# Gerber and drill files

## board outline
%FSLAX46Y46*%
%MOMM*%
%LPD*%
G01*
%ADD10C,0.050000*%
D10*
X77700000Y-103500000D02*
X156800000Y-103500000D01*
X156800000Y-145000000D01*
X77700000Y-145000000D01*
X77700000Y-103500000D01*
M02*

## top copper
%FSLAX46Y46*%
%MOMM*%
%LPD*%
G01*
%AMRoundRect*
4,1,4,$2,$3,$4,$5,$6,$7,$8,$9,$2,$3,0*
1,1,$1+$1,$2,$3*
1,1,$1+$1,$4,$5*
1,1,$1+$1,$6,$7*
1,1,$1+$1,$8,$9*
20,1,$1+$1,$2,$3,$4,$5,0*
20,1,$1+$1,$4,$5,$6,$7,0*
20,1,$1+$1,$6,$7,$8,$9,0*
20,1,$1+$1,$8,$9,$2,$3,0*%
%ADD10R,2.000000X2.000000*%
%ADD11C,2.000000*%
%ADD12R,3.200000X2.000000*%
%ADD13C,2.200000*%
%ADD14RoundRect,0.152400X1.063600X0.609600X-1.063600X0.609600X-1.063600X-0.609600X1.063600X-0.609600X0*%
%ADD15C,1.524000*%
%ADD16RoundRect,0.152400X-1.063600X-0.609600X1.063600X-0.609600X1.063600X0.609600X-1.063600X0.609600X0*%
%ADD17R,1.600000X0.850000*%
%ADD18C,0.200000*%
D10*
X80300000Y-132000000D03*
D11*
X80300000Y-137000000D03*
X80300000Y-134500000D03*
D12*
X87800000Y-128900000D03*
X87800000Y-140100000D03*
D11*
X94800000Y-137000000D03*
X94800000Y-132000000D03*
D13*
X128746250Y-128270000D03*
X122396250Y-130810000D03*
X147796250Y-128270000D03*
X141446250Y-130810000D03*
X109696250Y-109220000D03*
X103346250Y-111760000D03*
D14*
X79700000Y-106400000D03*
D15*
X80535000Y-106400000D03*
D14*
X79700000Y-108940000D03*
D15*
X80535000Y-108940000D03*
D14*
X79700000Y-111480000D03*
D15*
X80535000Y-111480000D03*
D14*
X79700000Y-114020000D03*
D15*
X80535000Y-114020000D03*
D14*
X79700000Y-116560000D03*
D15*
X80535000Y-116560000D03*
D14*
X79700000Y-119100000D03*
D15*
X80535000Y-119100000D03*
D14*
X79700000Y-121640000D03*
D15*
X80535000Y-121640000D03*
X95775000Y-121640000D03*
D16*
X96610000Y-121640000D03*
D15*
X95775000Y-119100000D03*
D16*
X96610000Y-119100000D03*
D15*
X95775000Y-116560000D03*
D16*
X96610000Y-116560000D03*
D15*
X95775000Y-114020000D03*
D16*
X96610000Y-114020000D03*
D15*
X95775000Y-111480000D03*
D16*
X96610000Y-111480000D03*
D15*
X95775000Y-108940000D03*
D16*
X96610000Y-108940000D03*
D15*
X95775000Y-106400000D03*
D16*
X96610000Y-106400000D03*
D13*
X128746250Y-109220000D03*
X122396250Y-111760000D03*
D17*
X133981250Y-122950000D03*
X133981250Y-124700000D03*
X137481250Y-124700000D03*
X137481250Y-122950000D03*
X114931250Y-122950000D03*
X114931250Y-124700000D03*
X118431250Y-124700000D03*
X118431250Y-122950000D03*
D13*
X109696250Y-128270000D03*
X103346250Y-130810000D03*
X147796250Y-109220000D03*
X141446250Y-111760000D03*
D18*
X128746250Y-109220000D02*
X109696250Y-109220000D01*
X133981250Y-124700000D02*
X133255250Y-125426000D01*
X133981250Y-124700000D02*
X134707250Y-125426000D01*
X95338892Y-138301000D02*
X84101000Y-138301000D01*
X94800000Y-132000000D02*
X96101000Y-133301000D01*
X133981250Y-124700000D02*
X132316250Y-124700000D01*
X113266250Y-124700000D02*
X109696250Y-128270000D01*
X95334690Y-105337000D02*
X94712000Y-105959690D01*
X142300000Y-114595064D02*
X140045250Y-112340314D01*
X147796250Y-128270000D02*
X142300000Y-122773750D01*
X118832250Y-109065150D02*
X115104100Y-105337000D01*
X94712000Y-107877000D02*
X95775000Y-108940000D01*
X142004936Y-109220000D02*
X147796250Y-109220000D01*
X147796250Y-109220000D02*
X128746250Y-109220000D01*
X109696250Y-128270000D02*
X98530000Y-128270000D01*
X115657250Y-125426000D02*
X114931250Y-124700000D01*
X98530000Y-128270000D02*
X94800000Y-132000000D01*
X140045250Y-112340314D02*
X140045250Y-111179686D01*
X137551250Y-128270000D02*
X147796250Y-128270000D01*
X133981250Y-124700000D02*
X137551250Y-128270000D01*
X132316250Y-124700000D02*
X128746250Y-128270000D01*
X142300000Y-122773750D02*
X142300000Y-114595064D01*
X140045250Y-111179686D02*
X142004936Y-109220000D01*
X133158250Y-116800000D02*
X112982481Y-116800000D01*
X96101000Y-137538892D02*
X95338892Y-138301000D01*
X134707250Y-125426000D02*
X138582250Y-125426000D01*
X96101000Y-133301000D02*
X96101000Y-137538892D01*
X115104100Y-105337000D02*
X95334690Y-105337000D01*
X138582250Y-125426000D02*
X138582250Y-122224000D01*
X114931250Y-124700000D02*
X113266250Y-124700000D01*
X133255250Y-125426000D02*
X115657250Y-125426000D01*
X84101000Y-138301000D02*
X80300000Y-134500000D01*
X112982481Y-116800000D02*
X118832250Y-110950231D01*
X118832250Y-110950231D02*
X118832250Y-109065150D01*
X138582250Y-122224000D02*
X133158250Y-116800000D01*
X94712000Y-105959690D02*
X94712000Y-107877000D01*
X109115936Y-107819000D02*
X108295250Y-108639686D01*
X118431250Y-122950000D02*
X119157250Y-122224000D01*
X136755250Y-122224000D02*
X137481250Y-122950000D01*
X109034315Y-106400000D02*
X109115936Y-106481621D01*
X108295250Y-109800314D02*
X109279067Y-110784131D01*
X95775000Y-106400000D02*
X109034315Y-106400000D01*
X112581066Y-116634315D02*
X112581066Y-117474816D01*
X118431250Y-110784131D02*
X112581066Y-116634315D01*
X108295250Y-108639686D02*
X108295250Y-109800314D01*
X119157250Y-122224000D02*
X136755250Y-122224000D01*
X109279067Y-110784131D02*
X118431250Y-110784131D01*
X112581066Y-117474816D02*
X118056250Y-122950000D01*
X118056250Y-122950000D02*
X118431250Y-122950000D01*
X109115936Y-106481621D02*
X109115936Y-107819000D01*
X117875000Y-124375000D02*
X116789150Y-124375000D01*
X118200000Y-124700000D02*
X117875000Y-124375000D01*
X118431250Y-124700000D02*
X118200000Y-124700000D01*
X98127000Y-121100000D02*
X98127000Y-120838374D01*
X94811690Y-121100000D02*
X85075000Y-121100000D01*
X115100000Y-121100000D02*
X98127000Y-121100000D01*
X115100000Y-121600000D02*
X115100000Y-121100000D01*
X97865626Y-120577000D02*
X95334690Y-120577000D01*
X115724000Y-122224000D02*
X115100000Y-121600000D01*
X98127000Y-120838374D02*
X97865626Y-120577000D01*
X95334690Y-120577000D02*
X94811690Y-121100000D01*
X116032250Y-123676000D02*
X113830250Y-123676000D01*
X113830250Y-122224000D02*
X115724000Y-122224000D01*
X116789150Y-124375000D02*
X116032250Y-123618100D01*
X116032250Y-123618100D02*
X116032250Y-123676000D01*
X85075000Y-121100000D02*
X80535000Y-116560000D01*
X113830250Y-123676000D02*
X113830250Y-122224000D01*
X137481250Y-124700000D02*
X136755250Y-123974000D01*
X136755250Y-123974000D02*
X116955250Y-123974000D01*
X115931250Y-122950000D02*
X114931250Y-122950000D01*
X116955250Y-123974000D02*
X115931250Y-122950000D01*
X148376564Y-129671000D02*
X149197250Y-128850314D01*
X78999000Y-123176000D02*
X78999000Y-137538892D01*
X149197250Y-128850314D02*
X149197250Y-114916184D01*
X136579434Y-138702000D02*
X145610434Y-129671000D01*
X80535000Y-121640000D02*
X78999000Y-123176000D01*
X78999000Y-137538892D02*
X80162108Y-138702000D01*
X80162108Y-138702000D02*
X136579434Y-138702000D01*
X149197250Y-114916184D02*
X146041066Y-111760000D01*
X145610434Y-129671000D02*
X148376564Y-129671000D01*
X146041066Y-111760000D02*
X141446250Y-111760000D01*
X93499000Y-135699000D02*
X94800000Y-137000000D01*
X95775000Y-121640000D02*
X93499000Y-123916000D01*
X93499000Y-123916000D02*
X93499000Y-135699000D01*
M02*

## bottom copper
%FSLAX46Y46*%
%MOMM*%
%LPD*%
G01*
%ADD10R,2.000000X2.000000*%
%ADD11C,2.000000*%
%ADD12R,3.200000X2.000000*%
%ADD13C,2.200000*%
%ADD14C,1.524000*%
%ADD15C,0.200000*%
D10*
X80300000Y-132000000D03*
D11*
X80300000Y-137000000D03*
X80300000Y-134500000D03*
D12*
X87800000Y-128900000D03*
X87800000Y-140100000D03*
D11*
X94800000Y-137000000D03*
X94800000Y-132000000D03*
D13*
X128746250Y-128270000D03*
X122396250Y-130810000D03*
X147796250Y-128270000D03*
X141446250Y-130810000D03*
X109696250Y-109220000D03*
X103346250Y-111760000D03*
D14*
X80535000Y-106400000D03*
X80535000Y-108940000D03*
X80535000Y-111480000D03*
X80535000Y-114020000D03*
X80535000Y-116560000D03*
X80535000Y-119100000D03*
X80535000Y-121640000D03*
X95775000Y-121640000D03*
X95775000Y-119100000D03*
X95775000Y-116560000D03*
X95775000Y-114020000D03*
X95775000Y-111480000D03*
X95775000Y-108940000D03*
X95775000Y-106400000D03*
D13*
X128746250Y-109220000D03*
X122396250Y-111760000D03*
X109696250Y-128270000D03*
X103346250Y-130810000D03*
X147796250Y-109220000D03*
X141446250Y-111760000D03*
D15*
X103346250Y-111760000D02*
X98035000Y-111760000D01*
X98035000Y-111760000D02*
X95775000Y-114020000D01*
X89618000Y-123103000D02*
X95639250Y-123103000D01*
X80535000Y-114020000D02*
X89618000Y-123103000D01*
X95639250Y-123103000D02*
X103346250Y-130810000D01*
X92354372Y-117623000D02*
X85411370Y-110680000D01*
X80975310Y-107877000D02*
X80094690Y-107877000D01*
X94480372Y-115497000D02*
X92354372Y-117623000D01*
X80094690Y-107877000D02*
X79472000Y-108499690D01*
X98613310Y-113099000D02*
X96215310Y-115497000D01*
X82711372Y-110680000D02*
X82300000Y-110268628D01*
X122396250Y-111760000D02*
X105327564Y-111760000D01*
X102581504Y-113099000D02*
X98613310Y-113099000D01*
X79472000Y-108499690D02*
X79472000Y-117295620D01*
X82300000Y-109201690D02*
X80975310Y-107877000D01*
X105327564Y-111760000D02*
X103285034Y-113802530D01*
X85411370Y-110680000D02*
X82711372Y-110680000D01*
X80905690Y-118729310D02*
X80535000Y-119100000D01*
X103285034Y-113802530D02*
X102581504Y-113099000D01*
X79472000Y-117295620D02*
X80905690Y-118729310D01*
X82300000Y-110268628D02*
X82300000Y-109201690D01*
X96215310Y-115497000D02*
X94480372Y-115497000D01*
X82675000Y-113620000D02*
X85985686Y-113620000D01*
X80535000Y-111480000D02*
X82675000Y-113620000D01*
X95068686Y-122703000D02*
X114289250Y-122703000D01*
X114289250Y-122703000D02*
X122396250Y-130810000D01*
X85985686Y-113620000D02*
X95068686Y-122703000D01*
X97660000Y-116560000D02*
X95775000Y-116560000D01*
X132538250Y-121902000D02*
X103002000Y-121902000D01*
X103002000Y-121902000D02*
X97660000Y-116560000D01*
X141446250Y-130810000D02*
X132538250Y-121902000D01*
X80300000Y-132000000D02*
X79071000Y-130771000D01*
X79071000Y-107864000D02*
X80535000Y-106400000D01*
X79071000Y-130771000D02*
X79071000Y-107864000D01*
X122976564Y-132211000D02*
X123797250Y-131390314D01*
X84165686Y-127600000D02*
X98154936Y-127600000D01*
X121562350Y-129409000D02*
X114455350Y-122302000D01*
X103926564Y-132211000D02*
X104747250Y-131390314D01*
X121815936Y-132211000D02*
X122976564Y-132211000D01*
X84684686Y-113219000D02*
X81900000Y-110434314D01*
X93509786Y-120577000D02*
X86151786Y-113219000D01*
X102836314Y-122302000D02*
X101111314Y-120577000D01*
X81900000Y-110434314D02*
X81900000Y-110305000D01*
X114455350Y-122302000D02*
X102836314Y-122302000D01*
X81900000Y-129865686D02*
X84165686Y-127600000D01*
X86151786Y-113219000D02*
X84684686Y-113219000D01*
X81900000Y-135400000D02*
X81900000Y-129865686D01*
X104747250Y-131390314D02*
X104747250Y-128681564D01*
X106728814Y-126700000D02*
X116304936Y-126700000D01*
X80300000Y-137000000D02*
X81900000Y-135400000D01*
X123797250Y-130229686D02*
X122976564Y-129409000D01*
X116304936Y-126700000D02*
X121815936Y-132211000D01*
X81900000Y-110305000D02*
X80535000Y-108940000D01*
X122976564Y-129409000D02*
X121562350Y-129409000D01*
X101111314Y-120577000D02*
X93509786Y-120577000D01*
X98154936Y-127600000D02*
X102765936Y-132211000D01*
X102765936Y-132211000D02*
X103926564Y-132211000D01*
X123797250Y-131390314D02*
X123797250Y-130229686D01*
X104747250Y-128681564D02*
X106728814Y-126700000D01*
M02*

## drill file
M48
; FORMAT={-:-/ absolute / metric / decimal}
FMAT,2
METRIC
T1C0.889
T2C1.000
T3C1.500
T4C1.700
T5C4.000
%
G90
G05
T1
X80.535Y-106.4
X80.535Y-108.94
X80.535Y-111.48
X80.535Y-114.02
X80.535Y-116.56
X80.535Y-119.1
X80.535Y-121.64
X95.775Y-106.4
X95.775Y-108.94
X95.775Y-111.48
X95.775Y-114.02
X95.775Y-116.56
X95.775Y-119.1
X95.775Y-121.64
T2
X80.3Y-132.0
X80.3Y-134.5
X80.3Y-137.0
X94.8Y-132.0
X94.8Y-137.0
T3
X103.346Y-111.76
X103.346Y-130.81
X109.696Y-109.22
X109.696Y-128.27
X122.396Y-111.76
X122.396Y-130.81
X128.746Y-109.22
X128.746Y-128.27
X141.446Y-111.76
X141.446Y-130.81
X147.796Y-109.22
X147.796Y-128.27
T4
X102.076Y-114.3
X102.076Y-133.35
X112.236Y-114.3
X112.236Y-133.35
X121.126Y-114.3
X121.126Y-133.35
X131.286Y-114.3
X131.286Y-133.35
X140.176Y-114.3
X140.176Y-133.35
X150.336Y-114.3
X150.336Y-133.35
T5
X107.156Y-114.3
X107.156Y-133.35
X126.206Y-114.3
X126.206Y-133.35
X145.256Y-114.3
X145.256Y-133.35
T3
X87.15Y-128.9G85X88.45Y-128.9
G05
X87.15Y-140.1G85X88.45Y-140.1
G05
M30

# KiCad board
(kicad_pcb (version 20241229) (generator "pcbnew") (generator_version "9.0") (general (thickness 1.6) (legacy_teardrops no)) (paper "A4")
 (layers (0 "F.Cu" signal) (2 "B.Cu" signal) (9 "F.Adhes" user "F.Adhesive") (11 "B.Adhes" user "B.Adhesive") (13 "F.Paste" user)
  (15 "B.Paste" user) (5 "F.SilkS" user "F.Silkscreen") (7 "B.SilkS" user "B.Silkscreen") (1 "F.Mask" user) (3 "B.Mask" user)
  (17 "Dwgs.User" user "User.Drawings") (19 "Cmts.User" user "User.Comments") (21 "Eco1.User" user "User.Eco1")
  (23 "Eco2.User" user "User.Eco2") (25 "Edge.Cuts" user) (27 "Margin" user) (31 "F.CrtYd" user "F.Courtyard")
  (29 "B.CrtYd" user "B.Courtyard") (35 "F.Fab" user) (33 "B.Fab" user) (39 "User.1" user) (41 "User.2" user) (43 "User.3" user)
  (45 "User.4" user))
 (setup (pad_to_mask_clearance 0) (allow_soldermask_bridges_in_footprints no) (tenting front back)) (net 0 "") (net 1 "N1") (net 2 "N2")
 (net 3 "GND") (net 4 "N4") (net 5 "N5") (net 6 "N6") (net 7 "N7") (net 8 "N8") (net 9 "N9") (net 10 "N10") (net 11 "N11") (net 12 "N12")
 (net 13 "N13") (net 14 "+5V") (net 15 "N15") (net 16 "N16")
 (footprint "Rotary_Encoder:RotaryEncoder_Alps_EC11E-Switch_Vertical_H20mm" (layer "F.Cu") (at 80.3 132)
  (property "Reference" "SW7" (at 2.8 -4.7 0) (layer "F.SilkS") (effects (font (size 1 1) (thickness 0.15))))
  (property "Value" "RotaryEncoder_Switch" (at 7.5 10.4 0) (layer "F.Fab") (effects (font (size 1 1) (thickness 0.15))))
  (pad "A" thru_hole rect (at 0 0) (size 2 2) (drill 1) (layers "*.Cu" "*.Mask") (remove_unused_layers no) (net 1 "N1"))
  (pad "B" thru_hole circle (at 0 5) (size 2 2) (drill 1) (layers "*.Cu" "*.Mask") (remove_unused_layers no) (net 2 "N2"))
  (pad "C" thru_hole circle (at 0 2.5) (size 2 2) (drill 1) (layers "*.Cu" "*.Mask") (remove_unused_layers no) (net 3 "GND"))
  (pad "MP" thru_hole rect (at 7.5 -3.1) (size 3.2 2) (drill oval 2.8 1.5) (layers "*.Cu" "*.Mask") (remove_unused_layers no))
  (pad "MP" thru_hole rect (at 7.5 8.1) (size 3.2 2) (drill oval 2.8 1.5) (layers "*.Cu" "*.Mask") (remove_unused_layers no))
  (pad "S1" thru_hole circle (at 14.5 5) (size 2 2) (drill 1) (layers "*.Cu" "*.Mask") (remove_unused_layers no) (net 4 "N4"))
  (pad "S2" thru_hole circle (at 14.5 0) (size 2 2) (drill 1) (layers "*.Cu" "*.Mask") (remove_unused_layers no) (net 3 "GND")))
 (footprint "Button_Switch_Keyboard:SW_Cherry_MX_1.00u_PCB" (layer "F.Cu") (at 128.74625 128.27)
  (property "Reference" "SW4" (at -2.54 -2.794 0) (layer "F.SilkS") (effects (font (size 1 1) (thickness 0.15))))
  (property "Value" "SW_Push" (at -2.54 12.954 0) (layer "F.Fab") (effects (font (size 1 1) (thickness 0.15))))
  (pad "" np_thru_hole circle (at -7.62 5.08) (size 1.7 1.7) (drill 1.7) (layers "*.Cu" "*.Mask"))
  (pad "" np_thru_hole circle (at -2.54 5.08) (size 4 4) (drill 4) (layers "*.Cu" "*.Mask"))
  (pad "" np_thru_hole circle (at 2.54 5.08) (size 1.7 1.7) (drill 1.7) (layers "*.Cu" "*.Mask"))
  (pad "1" thru_hole circle (at 0 0) (size 2.2 2.2) (drill 1.5) (layers "*.Cu" "*.Mask") (remove_unused_layers no) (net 3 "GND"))
  (pad "2" thru_hole circle (at -6.35 2.54) (size 2.2 2.2) (drill 1.5) (layers "*.Cu" "*.Mask") (remove_unused_layers no) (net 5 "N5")))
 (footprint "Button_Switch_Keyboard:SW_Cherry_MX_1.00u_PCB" (layer "F.Cu") (at 147.79625 128.27)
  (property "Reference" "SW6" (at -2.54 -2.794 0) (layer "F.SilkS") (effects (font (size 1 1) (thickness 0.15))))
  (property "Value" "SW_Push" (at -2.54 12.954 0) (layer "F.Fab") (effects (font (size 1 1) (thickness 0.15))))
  (pad "" np_thru_hole circle (at -7.62 5.08) (size 1.7 1.7) (drill 1.7) (layers "*.Cu" "*.Mask"))
  (pad "" np_thru_hole circle (at -2.54 5.08) (size 4 4) (drill 4) (layers "*.Cu" "*.Mask"))
  (pad "" np_thru_hole circle (at 2.54 5.08) (size 1.7 1.7) (drill 1.7) (layers "*.Cu" "*.Mask"))
  (pad "1" thru_hole circle (at 0 0) (size 2.2 2.2) (drill 1.5) (layers "*.Cu" "*.Mask") (remove_unused_layers no) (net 3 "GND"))
  (pad "2" thru_hole circle (at -6.35 2.54) (size 2.2 2.2) (drill 1.5) (layers "*.Cu" "*.Mask") (remove_unused_layers no) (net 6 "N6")))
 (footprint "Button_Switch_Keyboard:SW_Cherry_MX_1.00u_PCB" (layer "F.Cu") (at 109.69625 109.22)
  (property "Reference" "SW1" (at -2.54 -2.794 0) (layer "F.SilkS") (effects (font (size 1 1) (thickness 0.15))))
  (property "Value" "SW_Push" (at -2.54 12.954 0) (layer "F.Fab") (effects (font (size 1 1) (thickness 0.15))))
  (pad "" np_thru_hole circle (at -7.62 5.08) (size 1.7 1.7) (drill 1.7) (layers "*.Cu" "*.Mask"))
  (pad "" np_thru_hole circle (at -2.54 5.08) (size 4 4) (drill 4) (layers "*.Cu" "*.Mask"))
  (pad "" np_thru_hole circle (at 2.54 5.08) (size 1.7 1.7) (drill 1.7) (layers "*.Cu" "*.Mask"))
  (pad "1" thru_hole circle (at 0 0) (size 2.2 2.2) (drill 1.5) (layers "*.Cu" "*.Mask") (remove_unused_layers no) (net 3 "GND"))
  (pad "2" thru_hole circle (at -6.35 2.54) (size 2.2 2.2) (drill 1.5) (layers "*.Cu" "*.Mask") (remove_unused_layers no) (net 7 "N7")))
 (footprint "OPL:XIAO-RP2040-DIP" (layer "F.Cu") (at 88.155 114.02)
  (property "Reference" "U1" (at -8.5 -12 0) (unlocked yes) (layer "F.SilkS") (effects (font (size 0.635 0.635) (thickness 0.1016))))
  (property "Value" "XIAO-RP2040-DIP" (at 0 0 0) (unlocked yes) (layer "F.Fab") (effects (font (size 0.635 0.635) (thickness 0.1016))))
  (pad "1" smd roundrect (at -8.455 -7.62 180) (size 2.432 1.524) (layers "F.Cu" "F.Mask") (roundrect_rratio 0.1) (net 1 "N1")
   (thermal_bridge_angle 45))
  (pad "1" thru_hole circle (at -7.62 -7.62 180) (size 1.524 1.524) (drill 0.889) (layers "*.Cu" "*.Mask") (remove_unused_layers no)
   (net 1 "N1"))
  (pad "2" smd roundrect (at -8.455 -5.08 180) (size 2.432 1.524) (layers "F.Cu" "F.Mask") (roundrect_rratio 0.1) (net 2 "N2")
   (thermal_bridge_angle 45))
  (pad "2" thru_hole circle (at -7.62 -5.08 180) (size 1.524 1.524) (drill 0.889) (layers "*.Cu" "*.Mask") (remove_unused_layers no)
   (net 2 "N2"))
  (pad "3" smd roundrect (at -8.455 -2.54 180) (size 2.432 1.524) (layers "F.Cu" "F.Mask") (roundrect_rratio 0.1) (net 5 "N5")
   (thermal_bridge_angle 45))
  (pad "3" thru_hole circle (at -7.62 -2.54 180) (size 1.524 1.524) (drill 0.889) (layers "*.Cu" "*.Mask") (remove_unused_layers no)
   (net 5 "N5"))
  (pad "4" smd roundrect (at -8.455 0 180) (size 2.432 1.524) (layers "F.Cu" "F.Mask") (roundrect_rratio 0.1) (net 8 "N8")
   (thermal_bridge_angle 45))
  (pad "4" thru_hole circle (at -7.62 0 180) (size 1.524 1.524) (drill 0.889) (layers "*.Cu" "*.Mask") (remove_unused_layers no)
   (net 8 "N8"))
  (pad "5" smd roundrect (at -8.455 2.54 180) (size 2.432 1.524) (layers "F.Cu" "F.Mask") (roundrect_rratio 0.1) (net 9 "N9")
   (thermal_bridge_angle 45))
  (pad "5" thru_hole circle (at -7.62 2.54 180) (size 1.524 1.524) (drill 0.889) (layers "*.Cu" "*.Mask") (remove_unused_layers no)
   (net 9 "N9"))
  (pad "6" smd roundrect (at -8.455 5.08 180) (size 2.432 1.524) (layers "F.Cu" "F.Mask") (roundrect_rratio 0.1) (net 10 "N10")
   (thermal_bridge_angle 45))
  (pad "6" thru_hole circle (at -7.62 5.08 180) (size 1.524 1.524) (drill 0.889) (layers "*.Cu" "*.Mask") (remove_unused_layers no)
   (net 10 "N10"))
  (pad "7" smd roundrect (at -8.455 7.62 180) (size 2.432 1.524) (layers "F.Cu" "F.Mask") (roundrect_rratio 0.1) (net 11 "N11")
   (thermal_bridge_angle 45))
  (pad "7" thru_hole circle (at -7.62 7.62 180) (size 1.524 1.524) (drill 0.889) (layers "*.Cu" "*.Mask") (remove_unused_layers no)
   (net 11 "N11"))
  (pad "8" thru_hole circle (at 7.62 7.62) (size 1.524 1.524) (drill 0.889) (layers "*.Cu" "*.Mask") (remove_unused_layers no) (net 4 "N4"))
  (pad "8" smd roundrect (at 8.455 7.62) (size 2.432 1.524) (layers "F.Cu" "F.Mask") (roundrect_rratio 0.1) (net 4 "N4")
   (thermal_bridge_angle 45))
  (pad "9" thru_hole circle (at 7.62 5.08) (size 1.524 1.524) (drill 0.889) (layers "*.Cu" "*.Mask") (remove_unused_layers no)
   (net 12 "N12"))
  (pad "9" smd roundrect (at 8.455 5.08) (size 2.432 1.524) (layers "F.Cu" "F.Mask") (roundrect_rratio 0.1) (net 12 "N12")
   (thermal_bridge_angle 45))
  (pad "10" thru_hole circle (at 7.62 2.54) (size 1.524 1.524) (drill 0.889) (layers "*.Cu" "*.Mask") (remove_unused_layers no) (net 6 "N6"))
  (pad "10" smd roundrect (at 8.455 2.54) (size 2.432 1.524) (layers "F.Cu" "F.Mask") (roundrect_rratio 0.1) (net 6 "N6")
   (thermal_bridge_angle 45))
  (pad "11" thru_hole circle (at 7.62 0) (size 1.524 1.524) (drill 0.889) (layers "*.Cu" "*.Mask") (remove_unused_layers no) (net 7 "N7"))
  (pad "11" smd roundrect (at 8.455 0) (size 2.432 1.524) (layers "F.Cu" "F.Mask") (roundrect_rratio 0.1) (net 7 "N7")
   (thermal_bridge_angle 45))
  (pad "12" thru_hole circle (at 7.62 -2.54) (size 1.524 1.524) (drill 0.889) (layers "*.Cu" "*.Mask") (remove_unused_layers no)
   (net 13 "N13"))
  (pad "12" smd roundrect (at 8.455 -2.54) (size 2.432 1.524) (layers "F.Cu" "F.Mask") (roundrect_rratio 0.1) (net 13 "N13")
   (thermal_bridge_angle 45))
  (pad "13" thru_hole circle (at 7.62 -5.08) (size 1.524 1.524) (drill 0.889) (layers "*.Cu" "*.Mask") (remove_unused_layers no)
   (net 3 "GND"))
  (pad "13" smd roundrect (at 8.455 -5.08) (size 2.432 1.524) (layers "F.Cu" "F.Mask") (roundrect_rratio 0.1) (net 3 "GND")
   (thermal_bridge_angle 45))
  (pad "14" thru_hole circle (at 7.62 -7.62) (size 1.524 1.524) (drill 0.889) (layers "*.Cu" "*.Mask") (remove_unused_layers no)
   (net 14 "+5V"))
  (pad "14" smd roundrect (at 8.455 -7.62) (size 2.432 1.524) (layers "F.Cu" "F.Mask") (roundrect_rratio 0.1) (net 14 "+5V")
   (thermal_bridge_angle 45)))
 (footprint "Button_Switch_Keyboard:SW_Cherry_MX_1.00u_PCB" (layer "F.Cu") (at 128.74625 109.22)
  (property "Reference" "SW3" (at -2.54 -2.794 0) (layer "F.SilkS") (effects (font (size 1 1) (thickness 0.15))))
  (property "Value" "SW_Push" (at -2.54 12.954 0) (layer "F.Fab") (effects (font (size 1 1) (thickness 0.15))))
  (pad "" np_thru_hole circle (at -7.62 5.08) (size 1.7 1.7) (drill 1.7) (layers "*.Cu" "*.Mask"))
  (pad "" np_thru_hole circle (at -2.54 5.08) (size 4 4) (drill 4) (layers "*.Cu" "*.Mask"))
  (pad "" np_thru_hole circle (at 2.54 5.08) (size 1.7 1.7) (drill 1.7) (layers "*.Cu" "*.Mask"))
  (pad "1" thru_hole circle (at 0 0) (size 2.2 2.2) (drill 1.5) (layers "*.Cu" "*.Mask") (remove_unused_layers no) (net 3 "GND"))
  (pad "2" thru_hole circle (at -6.35 2.54) (size 2.2 2.2) (drill 1.5) (layers "*.Cu" "*.Mask") (remove_unused_layers no) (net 10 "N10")))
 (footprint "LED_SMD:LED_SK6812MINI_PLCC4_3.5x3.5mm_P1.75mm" (layer "F.Cu") (at 135.73125 123.825)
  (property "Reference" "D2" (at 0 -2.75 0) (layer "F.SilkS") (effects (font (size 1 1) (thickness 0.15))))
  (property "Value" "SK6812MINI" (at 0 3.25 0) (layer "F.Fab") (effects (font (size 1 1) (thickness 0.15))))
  (pad "1" smd rect (at -1.75 -0.875) (size 1.6 0.85) (layers "F.Cu" "F.Mask" "F.Paste") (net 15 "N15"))
  (pad "2" smd rect (at -1.75 0.875) (size 1.6 0.85) (layers "F.Cu" "F.Mask" "F.Paste") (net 3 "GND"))
  (pad "3" smd rect (at 1.75 0.875) (size 1.6 0.85) (layers "F.Cu" "F.Mask" "F.Paste") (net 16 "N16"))
  (pad "4" smd rect (at 1.75 -0.875) (size 1.6 0.85) (layers "F.Cu" "F.Mask" "F.Paste") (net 14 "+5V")))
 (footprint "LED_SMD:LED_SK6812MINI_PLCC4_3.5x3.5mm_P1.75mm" (layer "F.Cu") (at 116.68125 123.825)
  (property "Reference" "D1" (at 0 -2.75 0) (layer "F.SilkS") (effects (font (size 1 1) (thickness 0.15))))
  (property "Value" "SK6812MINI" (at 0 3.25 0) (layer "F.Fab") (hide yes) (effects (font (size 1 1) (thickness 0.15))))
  (pad "1" smd rect (at -1.75 -0.875) (size 1.6 0.85) (layers "F.Cu" "F.Mask" "F.Paste") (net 16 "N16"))
  (pad "2" smd rect (at -1.75 0.875) (size 1.6 0.85) (layers "F.Cu" "F.Mask" "F.Paste") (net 3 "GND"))
  (pad "3" smd rect (at 1.75 0.875) (size 1.6 0.85) (layers "F.Cu" "F.Mask" "F.Paste") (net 9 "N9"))
  (pad "4" smd rect (at 1.75 -0.875) (size 1.6 0.85) (layers "F.Cu" "F.Mask" "F.Paste") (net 14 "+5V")))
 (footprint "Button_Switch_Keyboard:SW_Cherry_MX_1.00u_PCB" (layer "F.Cu") (at 109.69625 128.27)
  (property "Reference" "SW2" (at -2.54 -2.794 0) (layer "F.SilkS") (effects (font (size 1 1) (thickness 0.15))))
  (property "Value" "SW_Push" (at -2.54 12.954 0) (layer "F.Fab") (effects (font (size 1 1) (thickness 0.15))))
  (pad "" np_thru_hole circle (at -7.62 5.08) (size 1.7 1.7) (drill 1.7) (layers "*.Cu" "*.Mask"))
  (pad "" np_thru_hole circle (at -2.54 5.08) (size 4 4) (drill 4) (layers "*.Cu" "*.Mask"))
  (pad "" np_thru_hole circle (at 2.54 5.08) (size 1.7 1.7) (drill 1.7) (layers "*.Cu" "*.Mask"))
  (pad "1" thru_hole circle (at 0 0) (size 2.2 2.2) (drill 1.5) (layers "*.Cu" "*.Mask") (remove_unused_layers no) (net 3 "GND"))
  (pad "2" thru_hole circle (at -6.35 2.54) (size 2.2 2.2) (drill 1.5) (layers "*.Cu" "*.Mask") (remove_unused_layers no) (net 8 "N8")))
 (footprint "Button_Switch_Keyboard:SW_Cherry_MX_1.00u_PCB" (layer "F.Cu") (at 147.79625 109.22)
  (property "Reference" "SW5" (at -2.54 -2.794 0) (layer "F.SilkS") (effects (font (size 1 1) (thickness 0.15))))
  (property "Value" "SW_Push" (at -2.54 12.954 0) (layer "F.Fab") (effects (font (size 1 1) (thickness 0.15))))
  (pad "" np_thru_hole circle (at -7.62 5.08) (size 1.7 1.7) (drill 1.7) (layers "*.Cu" "*.Mask"))
  (pad "" np_thru_hole circle (at -2.54 5.08) (size 4 4) (drill 4) (layers "*.Cu" "*.Mask"))
  (pad "" np_thru_hole circle (at 2.54 5.08) (size 1.7 1.7) (drill 1.7) (layers "*.Cu" "*.Mask"))
  (pad "1" thru_hole circle (at 0 0) (size 2.2 2.2) (drill 1.5) (layers "*.Cu" "*.Mask") (remove_unused_layers no) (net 3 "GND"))
  (pad "2" thru_hole circle (at -6.35 2.54) (size 2.2 2.2) (drill 1.5) (layers "*.Cu" "*.Mask") (remove_unused_layers no) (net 11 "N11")))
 (gr_rect (start 77.7 103.5) (end 156.8 145) (stroke (width 0.05) (type default)) (fill no) (layer "Edge.Cuts"))
 (segment (start 128.74625 109.22) (end 109.69625 109.22) (width 0.2) (layer "F.Cu") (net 3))
 (segment (start 133.98125 124.7) (end 133.25525 125.426) (width 0.2) (layer "F.Cu") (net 3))
 (segment (start 133.98125 124.7) (end 134.70725 125.426) (width 0.2) (layer "F.Cu") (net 3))
 (segment (start 95.338892 138.301) (end 84.101 138.301) (width 0.2) (layer "F.Cu") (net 3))
 (segment (start 94.8 132) (end 96.101 133.301) (width 0.2) (layer "F.Cu") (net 3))
 (segment (start 133.98125 124.7) (end 132.31625 124.7) (width 0.2) (layer "F.Cu") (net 3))
 (segment (start 113.26625 124.7) (end 109.69625 128.27) (width 0.2) (layer "F.Cu") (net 3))
 (segment (start 95.33469 105.337) (end 94.712 105.95969) (width 0.2) (layer "F.Cu") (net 3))
 (segment (start 142.3 114.595064) (end 140.04525 112.340314) (width 0.2) (layer "F.Cu") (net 3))
 (segment (start 147.79625 128.27) (end 142.3 122.77375) (width 0.2) (layer "F.Cu") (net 3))
 (segment (start 118.83225 109.06515) (end 115.1041 105.337) (width 0.2) (layer "F.Cu") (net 3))
 (segment (start 94.712 107.877) (end 95.775 108.94) (width 0.2) (layer "F.Cu") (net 3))
 (segment (start 142.004936 109.22) (end 147.79625 109.22) (width 0.2) (layer "F.Cu") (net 3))
 (segment (start 147.79625 109.22) (end 128.74625 109.22) (width 0.2) (layer "F.Cu") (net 3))
 (segment (start 109.69625 128.27) (end 98.53 128.27) (width 0.2) (layer "F.Cu") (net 3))
 (segment (start 115.65725 125.426) (end 114.93125 124.7) (width 0.2) (layer "F.Cu") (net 3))
 (segment (start 98.53 128.27) (end 94.8 132) (width 0.2) (layer "F.Cu") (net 3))
 (segment (start 140.04525 112.340314) (end 140.04525 111.179686) (width 0.2) (layer "F.Cu") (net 3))
 (segment (start 137.55125 128.27) (end 147.79625 128.27) (width 0.2) (layer "F.Cu") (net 3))
 (segment (start 133.98125 124.7) (end 137.55125 128.27) (width 0.2) (layer "F.Cu") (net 3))
 (segment (start 132.31625 124.7) (end 128.74625 128.27) (width 0.2) (layer "F.Cu") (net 3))
 (segment (start 142.3 122.77375) (end 142.3 114.595064) (width 0.2) (layer "F.Cu") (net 3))
 (segment (start 140.04525 111.179686) (end 142.004936 109.22) (width 0.2) (layer "F.Cu") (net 3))
 (segment (start 133.15825 116.8) (end 112.982481 116.8) (width 0.2) (layer "F.Cu") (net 3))
 (segment (start 96.101 137.538892) (end 95.338892 138.301) (width 0.2) (layer "F.Cu") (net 3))
 (segment (start 134.70725 125.426) (end 138.58225 125.426) (width 0.2) (layer "F.Cu") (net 3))
 (segment (start 96.101 133.301) (end 96.101 137.538892) (width 0.2) (layer "F.Cu") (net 3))
 (segment (start 115.1041 105.337) (end 95.33469 105.337) (width 0.2) (layer "F.Cu") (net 3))
 (segment (start 138.58225 125.426) (end 138.58225 122.224) (width 0.2) (layer "F.Cu") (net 3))
 (segment (start 114.93125 124.7) (end 113.26625 124.7) (width 0.2) (layer "F.Cu") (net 3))
 (segment (start 133.25525 125.426) (end 115.65725 125.426) (width 0.2) (layer "F.Cu") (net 3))
 (segment (start 84.101 138.301) (end 80.3 134.5) (width 0.2) (layer "F.Cu") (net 3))
 (segment (start 112.982481 116.8) (end 118.83225 110.950231) (width 0.2) (layer "F.Cu") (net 3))
 (segment (start 118.83225 110.950231) (end 118.83225 109.06515) (width 0.2) (layer "F.Cu") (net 3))
 (segment (start 138.58225 122.224) (end 133.15825 116.8) (width 0.2) (layer "F.Cu") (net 3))
 (segment (start 94.712 105.95969) (end 94.712 107.877) (width 0.2) (layer "F.Cu") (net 3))
 (segment (start 109.115936 107.819) (end 108.29525 108.639686) (width 0.2) (layer "F.Cu") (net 14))
 (segment (start 118.43125 122.95) (end 119.15725 122.224) (width 0.2) (layer "F.Cu") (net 14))
 (segment (start 136.75525 122.224) (end 137.48125 122.95) (width 0.2) (layer "F.Cu") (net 14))
 (segment (start 109.034315 106.4) (end 109.115936 106.481621) (width 0.2) (layer "F.Cu") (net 14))
 (segment (start 108.29525 109.800314) (end 109.279067 110.784131) (width 0.2) (layer "F.Cu") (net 14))
 (segment (start 95.775 106.4) (end 109.034315 106.4) (width 0.2) (layer "F.Cu") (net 14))
 (segment (start 112.581066 116.634315) (end 112.581066 117.474816) (width 0.2) (layer "F.Cu") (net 14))
 (segment (start 118.43125 110.784131) (end 112.581066 116.634315) (width 0.2) (layer "F.Cu") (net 14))
 (segment (start 108.29525 108.639686) (end 108.29525 109.800314) (width 0.2) (layer "F.Cu") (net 14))
 (segment (start 119.15725 122.224) (end 136.75525 122.224) (width 0.2) (layer "F.Cu") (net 14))
 (segment (start 109.279067 110.784131) (end 118.43125 110.784131) (width 0.2) (layer "F.Cu") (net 14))
 (segment (start 112.581066 117.474816) (end 118.05625 122.95) (width 0.2) (layer "F.Cu") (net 14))
 (segment (start 118.05625 122.95) (end 118.43125 122.95) (width 0.2) (layer "F.Cu") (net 14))
 (segment (start 109.115936 106.481621) (end 109.115936 107.819) (width 0.2) (layer "F.Cu") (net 14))
 (segment (start 117.875 124.375) (end 116.78915 124.375) (width 0.2) (layer "F.Cu") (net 9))
 (segment (start 118.2 124.7) (end 117.875 124.375) (width 0.2) (layer "F.Cu") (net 9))
 (segment (start 118.43125 124.7) (end 118.2 124.7) (width 0.2) (layer "F.Cu") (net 9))
 (segment (start 98.127 121.1) (end 98.127 120.838374) (width 0.2) (layer "F.Cu") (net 9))
 (segment (start 94.81169 121.1) (end 85.075 121.1) (width 0.2) (layer "F.Cu") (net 9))
 (segment (start 115.1 121.1) (end 98.127 121.1) (width 0.2) (layer "F.Cu") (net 9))
 (segment (start 115.1 121.6) (end 115.1 121.1) (width 0.2) (layer "F.Cu") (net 9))
 (segment (start 97.865626 120.577) (end 95.33469 120.577) (width 0.2) (layer "F.Cu") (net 9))
 (segment (start 115.724 122.224) (end 115.1 121.6) (width 0.2) (layer "F.Cu") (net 9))
 (segment (start 98.127 120.838374) (end 97.865626 120.577) (width 0.2) (layer "F.Cu") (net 9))
 (segment (start 95.33469 120.577) (end 94.81169 121.1) (width 0.2) (layer "F.Cu") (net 9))
 (segment (start 116.03225 123.676) (end 113.83025 123.676) (width 0.2) (layer "F.Cu") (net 9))
 (segment (start 113.83025 122.224) (end 115.724 122.224) (width 0.2) (layer "F.Cu") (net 9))
 (segment (start 116.78915 124.375) (end 116.03225 123.6181) (width 0.2) (layer "F.Cu") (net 9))
 (segment (start 116.03225 123.6181) (end 116.03225 123.676) (width 0.2) (layer "F.Cu") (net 9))
 (segment (start 85.075 121.1) (end 80.535 116.56) (width 0.2) (layer "F.Cu") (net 9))
 (segment (start 113.83025 123.676) (end 113.83025 122.224) (width 0.2) (layer "F.Cu") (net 9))
 (segment (start 137.48125 124.7) (end 136.75525 123.974) (width 0.2) (layer "F.Cu") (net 16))
 (segment (start 136.75525 123.974) (end 116.95525 123.974) (width 0.2) (layer "F.Cu") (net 16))
 (segment (start 115.93125 122.95) (end 114.93125 122.95) (width 0.2) (layer "F.Cu") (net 16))
 (segment (start 116.95525 123.974) (end 115.93125 122.95) (width 0.2) (layer "F.Cu") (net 16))
 (segment (start 103.34625 111.76) (end 98.035 111.76) (width 0.2) (layer "B.Cu") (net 7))
 (segment (start 98.035 111.76) (end 95.775 114.02) (width 0.2) (layer "B.Cu") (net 7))
 (segment (start 89.618 123.103) (end 95.63925 123.103) (width 0.2) (layer "B.Cu") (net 8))
 (segment (start 80.535 114.02) (end 89.618 123.103) (width 0.2) (layer "B.Cu") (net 8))
 (segment (start 95.63925 123.103) (end 103.34625 130.81) (width 0.2) (layer "B.Cu") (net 8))
 (segment (start 92.354372 117.623) (end 85.41137 110.68) (width 0.2) (layer "B.Cu") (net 10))
 (segment (start 80.97531 107.877) (end 80.09469 107.877) (width 0.2) (layer "B.Cu") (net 10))
 (segment (start 94.480372 115.497) (end 92.354372 117.623) (width 0.2) (layer "B.Cu") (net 10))
 (segment (start 80.09469 107.877) (end 79.472 108.49969) (width 0.2) (layer "B.Cu") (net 10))
 (segment (start 98.61331 113.099) (end 96.21531 115.497) (width 0.2) (layer "B.Cu") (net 10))
 (segment (start 82.711372 110.68) (end 82.3 110.268628) (width 0.2) (layer "B.Cu") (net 10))
 (segment (start 122.39625 111.76) (end 105.327564 111.76) (width 0.2) (layer "B.Cu") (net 10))
 (segment (start 102.581504 113.099) (end 98.61331 113.099) (width 0.2) (layer "B.Cu") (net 10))
 (segment (start 79.472 108.49969) (end 79.472 117.29562) (width 0.2) (layer "B.Cu") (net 10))
 (segment (start 82.3 109.20169) (end 80.97531 107.877) (width 0.2) (layer "B.Cu") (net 10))
 (segment (start 105.327564 111.76) (end 103.285034 113.80253) (width 0.2) (layer "B.Cu") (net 10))
 (segment (start 85.41137 110.68) (end 82.711372 110.68) (width 0.2) (layer "B.Cu") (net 10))
 (segment (start 80.90569 118.72931) (end 80.535 119.1) (width 0.2) (layer "B.Cu") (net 10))
 (segment (start 103.285034 113.80253) (end 102.581504 113.099) (width 0.2) (layer "B.Cu") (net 10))
 (segment (start 79.472 117.29562) (end 80.90569 118.72931) (width 0.2) (layer "B.Cu") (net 10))
 (segment (start 82.3 110.268628) (end 82.3 109.20169) (width 0.2) (layer "B.Cu") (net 10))
 (segment (start 96.21531 115.497) (end 94.480372 115.497) (width 0.2) (layer "B.Cu") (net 10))
 (segment (start 82.675 113.62) (end 85.985686 113.62) (width 0.2) (layer "B.Cu") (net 5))
 (segment (start 80.535 111.48) (end 82.675 113.62) (width 0.2) (layer "B.Cu") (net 5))
 (segment (start 95.068686 122.703) (end 114.28925 122.703) (width 0.2) (layer "B.Cu") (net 5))
 (segment (start 114.28925 122.703) (end 122.39625 130.81) (width 0.2) (layer "B.Cu") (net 5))
 (segment (start 85.985686 113.62) (end 95.068686 122.703) (width 0.2) (layer "B.Cu") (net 5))
 (segment (start 148.376564 129.671) (end 149.19725 128.850314) (width 0.2) (layer "F.Cu") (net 11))
 (segment (start 78.999 123.176) (end 78.999 137.538892) (width 0.2) (layer "F.Cu") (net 11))
 (segment (start 149.19725 128.850314) (end 149.19725 114.916184) (width 0.2) (layer "F.Cu") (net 11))
 (segment (start 136.579434 138.702) (end 145.610434 129.671) (width 0.2) (layer "F.Cu") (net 11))
 (segment (start 80.535 121.64) (end 78.999 123.176) (width 0.2) (layer "F.Cu") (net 11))
 (segment (start 78.999 137.538892) (end 80.162108 138.702) (width 0.2) (layer "F.Cu") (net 11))
 (segment (start 80.162108 138.702) (end 136.579434 138.702) (width 0.2) (layer "F.Cu") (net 11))
 (segment (start 149.19725 114.916184) (end 146.041066 111.76) (width 0.2) (layer "F.Cu") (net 11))
 (segment (start 145.610434 129.671) (end 148.376564 129.671) (width 0.2) (layer "F.Cu") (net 11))
 (segment (start 146.041066 111.76) (end 141.44625 111.76) (width 0.2) (layer "F.Cu") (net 11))
 (segment (start 97.66 116.56) (end 95.775 116.56) (width 0.2) (layer "B.Cu") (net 6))
 (segment (start 132.53825 121.902) (end 103.002 121.902) (width 0.2) (layer "B.Cu") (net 6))
 (segment (start 103.002 121.902) (end 97.66 116.56) (width 0.2) (layer "B.Cu") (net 6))
 (segment (start 141.44625 130.81) (end 132.53825 121.902) (width 0.2) (layer "B.Cu") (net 6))
 (segment (start 80.3 132) (end 79.071 130.771) (width 0.2) (layer "B.Cu") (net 1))
 (segment (start 79.071 107.864) (end 80.535 106.4) (width 0.2) (layer "B.Cu") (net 1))
 (segment (start 79.071 130.771) (end 79.071 107.864) (width 0.2) (layer "B.Cu") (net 1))
 (segment (start 122.976564 132.211) (end 123.79725 131.390314) (width 0.2) (layer "B.Cu") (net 2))
 (segment (start 84.165686 127.6) (end 98.154936 127.6) (width 0.2) (layer "B.Cu") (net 2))
 (segment (start 121.56235 129.409) (end 114.45535 122.302) (width 0.2) (layer "B.Cu") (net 2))
 (segment (start 103.926564 132.211) (end 104.74725 131.390314) (width 0.2) (layer "B.Cu") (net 2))
 (segment (start 121.815936 132.211) (end 122.976564 132.211) (width 0.2) (layer "B.Cu") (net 2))
 (segment (start 84.684686 113.219) (end 81.9 110.434314) (width 0.2) (layer "B.Cu") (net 2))
 (segment (start 93.509786 120.577) (end 86.151786 113.219) (width 0.2) (layer "B.Cu") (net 2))
 (segment (start 102.836314 122.302) (end 101.111314 120.577) (width 0.2) (layer "B.Cu") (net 2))
 (segment (start 81.9 110.434314) (end 81.9 110.305) (width 0.2) (layer "B.Cu") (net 2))
 (segment (start 114.45535 122.302) (end 102.836314 122.302) (width 0.2) (layer "B.Cu") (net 2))
 (segment (start 81.9 129.865686) (end 84.165686 127.6) (width 0.2) (layer "B.Cu") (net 2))
 (segment (start 86.151786 113.219) (end 84.684686 113.219) (width 0.2) (layer "B.Cu") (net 2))
 (segment (start 81.9 135.4) (end 81.9 129.865686) (width 0.2) (layer "B.Cu") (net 2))
 (segment (start 104.74725 131.390314) (end 104.74725 128.681564) (width 0.2) (layer "B.Cu") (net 2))
 (segment (start 106.728814 126.7) (end 116.304936 126.7) (width 0.2) (layer "B.Cu") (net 2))
 (segment (start 80.3 137) (end 81.9 135.4) (width 0.2) (layer "B.Cu") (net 2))
 (segment (start 123.79725 130.229686) (end 122.976564 129.409) (width 0.2) (layer "B.Cu") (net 2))
 (segment (start 116.304936 126.7) (end 121.815936 132.211) (width 0.2) (layer "B.Cu") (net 2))
 (segment (start 81.9 110.305) (end 80.535 108.94) (width 0.2) (layer "B.Cu") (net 2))
 (segment (start 122.976564 129.409) (end 121.56235 129.409) (width 0.2) (layer "B.Cu") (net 2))
 (segment (start 101.111314 120.577) (end 93.509786 120.577) (width 0.2) (layer "B.Cu") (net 2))
 (segment (start 98.154936 127.6) (end 102.765936 132.211) (width 0.2) (layer "B.Cu") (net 2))
 (segment (start 102.765936 132.211) (end 103.926564 132.211) (width 0.2) (layer "B.Cu") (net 2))
 (segment (start 123.79725 131.390314) (end 123.79725 130.229686) (width 0.2) (layer "B.Cu") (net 2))
 (segment (start 104.74725 128.681564) (end 106.728814 126.7) (width 0.2) (layer "B.Cu") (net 2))
 (segment (start 93.499 135.699) (end 94.8 137) (width 0.2) (layer "F.Cu") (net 4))
 (segment (start 95.775 121.64) (end 93.499 123.916) (width 0.2) (layer "F.Cu") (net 4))
 (segment (start 93.499 123.916) (end 93.499 135.699) (width 0.2) (layer "F.Cu") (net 4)))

